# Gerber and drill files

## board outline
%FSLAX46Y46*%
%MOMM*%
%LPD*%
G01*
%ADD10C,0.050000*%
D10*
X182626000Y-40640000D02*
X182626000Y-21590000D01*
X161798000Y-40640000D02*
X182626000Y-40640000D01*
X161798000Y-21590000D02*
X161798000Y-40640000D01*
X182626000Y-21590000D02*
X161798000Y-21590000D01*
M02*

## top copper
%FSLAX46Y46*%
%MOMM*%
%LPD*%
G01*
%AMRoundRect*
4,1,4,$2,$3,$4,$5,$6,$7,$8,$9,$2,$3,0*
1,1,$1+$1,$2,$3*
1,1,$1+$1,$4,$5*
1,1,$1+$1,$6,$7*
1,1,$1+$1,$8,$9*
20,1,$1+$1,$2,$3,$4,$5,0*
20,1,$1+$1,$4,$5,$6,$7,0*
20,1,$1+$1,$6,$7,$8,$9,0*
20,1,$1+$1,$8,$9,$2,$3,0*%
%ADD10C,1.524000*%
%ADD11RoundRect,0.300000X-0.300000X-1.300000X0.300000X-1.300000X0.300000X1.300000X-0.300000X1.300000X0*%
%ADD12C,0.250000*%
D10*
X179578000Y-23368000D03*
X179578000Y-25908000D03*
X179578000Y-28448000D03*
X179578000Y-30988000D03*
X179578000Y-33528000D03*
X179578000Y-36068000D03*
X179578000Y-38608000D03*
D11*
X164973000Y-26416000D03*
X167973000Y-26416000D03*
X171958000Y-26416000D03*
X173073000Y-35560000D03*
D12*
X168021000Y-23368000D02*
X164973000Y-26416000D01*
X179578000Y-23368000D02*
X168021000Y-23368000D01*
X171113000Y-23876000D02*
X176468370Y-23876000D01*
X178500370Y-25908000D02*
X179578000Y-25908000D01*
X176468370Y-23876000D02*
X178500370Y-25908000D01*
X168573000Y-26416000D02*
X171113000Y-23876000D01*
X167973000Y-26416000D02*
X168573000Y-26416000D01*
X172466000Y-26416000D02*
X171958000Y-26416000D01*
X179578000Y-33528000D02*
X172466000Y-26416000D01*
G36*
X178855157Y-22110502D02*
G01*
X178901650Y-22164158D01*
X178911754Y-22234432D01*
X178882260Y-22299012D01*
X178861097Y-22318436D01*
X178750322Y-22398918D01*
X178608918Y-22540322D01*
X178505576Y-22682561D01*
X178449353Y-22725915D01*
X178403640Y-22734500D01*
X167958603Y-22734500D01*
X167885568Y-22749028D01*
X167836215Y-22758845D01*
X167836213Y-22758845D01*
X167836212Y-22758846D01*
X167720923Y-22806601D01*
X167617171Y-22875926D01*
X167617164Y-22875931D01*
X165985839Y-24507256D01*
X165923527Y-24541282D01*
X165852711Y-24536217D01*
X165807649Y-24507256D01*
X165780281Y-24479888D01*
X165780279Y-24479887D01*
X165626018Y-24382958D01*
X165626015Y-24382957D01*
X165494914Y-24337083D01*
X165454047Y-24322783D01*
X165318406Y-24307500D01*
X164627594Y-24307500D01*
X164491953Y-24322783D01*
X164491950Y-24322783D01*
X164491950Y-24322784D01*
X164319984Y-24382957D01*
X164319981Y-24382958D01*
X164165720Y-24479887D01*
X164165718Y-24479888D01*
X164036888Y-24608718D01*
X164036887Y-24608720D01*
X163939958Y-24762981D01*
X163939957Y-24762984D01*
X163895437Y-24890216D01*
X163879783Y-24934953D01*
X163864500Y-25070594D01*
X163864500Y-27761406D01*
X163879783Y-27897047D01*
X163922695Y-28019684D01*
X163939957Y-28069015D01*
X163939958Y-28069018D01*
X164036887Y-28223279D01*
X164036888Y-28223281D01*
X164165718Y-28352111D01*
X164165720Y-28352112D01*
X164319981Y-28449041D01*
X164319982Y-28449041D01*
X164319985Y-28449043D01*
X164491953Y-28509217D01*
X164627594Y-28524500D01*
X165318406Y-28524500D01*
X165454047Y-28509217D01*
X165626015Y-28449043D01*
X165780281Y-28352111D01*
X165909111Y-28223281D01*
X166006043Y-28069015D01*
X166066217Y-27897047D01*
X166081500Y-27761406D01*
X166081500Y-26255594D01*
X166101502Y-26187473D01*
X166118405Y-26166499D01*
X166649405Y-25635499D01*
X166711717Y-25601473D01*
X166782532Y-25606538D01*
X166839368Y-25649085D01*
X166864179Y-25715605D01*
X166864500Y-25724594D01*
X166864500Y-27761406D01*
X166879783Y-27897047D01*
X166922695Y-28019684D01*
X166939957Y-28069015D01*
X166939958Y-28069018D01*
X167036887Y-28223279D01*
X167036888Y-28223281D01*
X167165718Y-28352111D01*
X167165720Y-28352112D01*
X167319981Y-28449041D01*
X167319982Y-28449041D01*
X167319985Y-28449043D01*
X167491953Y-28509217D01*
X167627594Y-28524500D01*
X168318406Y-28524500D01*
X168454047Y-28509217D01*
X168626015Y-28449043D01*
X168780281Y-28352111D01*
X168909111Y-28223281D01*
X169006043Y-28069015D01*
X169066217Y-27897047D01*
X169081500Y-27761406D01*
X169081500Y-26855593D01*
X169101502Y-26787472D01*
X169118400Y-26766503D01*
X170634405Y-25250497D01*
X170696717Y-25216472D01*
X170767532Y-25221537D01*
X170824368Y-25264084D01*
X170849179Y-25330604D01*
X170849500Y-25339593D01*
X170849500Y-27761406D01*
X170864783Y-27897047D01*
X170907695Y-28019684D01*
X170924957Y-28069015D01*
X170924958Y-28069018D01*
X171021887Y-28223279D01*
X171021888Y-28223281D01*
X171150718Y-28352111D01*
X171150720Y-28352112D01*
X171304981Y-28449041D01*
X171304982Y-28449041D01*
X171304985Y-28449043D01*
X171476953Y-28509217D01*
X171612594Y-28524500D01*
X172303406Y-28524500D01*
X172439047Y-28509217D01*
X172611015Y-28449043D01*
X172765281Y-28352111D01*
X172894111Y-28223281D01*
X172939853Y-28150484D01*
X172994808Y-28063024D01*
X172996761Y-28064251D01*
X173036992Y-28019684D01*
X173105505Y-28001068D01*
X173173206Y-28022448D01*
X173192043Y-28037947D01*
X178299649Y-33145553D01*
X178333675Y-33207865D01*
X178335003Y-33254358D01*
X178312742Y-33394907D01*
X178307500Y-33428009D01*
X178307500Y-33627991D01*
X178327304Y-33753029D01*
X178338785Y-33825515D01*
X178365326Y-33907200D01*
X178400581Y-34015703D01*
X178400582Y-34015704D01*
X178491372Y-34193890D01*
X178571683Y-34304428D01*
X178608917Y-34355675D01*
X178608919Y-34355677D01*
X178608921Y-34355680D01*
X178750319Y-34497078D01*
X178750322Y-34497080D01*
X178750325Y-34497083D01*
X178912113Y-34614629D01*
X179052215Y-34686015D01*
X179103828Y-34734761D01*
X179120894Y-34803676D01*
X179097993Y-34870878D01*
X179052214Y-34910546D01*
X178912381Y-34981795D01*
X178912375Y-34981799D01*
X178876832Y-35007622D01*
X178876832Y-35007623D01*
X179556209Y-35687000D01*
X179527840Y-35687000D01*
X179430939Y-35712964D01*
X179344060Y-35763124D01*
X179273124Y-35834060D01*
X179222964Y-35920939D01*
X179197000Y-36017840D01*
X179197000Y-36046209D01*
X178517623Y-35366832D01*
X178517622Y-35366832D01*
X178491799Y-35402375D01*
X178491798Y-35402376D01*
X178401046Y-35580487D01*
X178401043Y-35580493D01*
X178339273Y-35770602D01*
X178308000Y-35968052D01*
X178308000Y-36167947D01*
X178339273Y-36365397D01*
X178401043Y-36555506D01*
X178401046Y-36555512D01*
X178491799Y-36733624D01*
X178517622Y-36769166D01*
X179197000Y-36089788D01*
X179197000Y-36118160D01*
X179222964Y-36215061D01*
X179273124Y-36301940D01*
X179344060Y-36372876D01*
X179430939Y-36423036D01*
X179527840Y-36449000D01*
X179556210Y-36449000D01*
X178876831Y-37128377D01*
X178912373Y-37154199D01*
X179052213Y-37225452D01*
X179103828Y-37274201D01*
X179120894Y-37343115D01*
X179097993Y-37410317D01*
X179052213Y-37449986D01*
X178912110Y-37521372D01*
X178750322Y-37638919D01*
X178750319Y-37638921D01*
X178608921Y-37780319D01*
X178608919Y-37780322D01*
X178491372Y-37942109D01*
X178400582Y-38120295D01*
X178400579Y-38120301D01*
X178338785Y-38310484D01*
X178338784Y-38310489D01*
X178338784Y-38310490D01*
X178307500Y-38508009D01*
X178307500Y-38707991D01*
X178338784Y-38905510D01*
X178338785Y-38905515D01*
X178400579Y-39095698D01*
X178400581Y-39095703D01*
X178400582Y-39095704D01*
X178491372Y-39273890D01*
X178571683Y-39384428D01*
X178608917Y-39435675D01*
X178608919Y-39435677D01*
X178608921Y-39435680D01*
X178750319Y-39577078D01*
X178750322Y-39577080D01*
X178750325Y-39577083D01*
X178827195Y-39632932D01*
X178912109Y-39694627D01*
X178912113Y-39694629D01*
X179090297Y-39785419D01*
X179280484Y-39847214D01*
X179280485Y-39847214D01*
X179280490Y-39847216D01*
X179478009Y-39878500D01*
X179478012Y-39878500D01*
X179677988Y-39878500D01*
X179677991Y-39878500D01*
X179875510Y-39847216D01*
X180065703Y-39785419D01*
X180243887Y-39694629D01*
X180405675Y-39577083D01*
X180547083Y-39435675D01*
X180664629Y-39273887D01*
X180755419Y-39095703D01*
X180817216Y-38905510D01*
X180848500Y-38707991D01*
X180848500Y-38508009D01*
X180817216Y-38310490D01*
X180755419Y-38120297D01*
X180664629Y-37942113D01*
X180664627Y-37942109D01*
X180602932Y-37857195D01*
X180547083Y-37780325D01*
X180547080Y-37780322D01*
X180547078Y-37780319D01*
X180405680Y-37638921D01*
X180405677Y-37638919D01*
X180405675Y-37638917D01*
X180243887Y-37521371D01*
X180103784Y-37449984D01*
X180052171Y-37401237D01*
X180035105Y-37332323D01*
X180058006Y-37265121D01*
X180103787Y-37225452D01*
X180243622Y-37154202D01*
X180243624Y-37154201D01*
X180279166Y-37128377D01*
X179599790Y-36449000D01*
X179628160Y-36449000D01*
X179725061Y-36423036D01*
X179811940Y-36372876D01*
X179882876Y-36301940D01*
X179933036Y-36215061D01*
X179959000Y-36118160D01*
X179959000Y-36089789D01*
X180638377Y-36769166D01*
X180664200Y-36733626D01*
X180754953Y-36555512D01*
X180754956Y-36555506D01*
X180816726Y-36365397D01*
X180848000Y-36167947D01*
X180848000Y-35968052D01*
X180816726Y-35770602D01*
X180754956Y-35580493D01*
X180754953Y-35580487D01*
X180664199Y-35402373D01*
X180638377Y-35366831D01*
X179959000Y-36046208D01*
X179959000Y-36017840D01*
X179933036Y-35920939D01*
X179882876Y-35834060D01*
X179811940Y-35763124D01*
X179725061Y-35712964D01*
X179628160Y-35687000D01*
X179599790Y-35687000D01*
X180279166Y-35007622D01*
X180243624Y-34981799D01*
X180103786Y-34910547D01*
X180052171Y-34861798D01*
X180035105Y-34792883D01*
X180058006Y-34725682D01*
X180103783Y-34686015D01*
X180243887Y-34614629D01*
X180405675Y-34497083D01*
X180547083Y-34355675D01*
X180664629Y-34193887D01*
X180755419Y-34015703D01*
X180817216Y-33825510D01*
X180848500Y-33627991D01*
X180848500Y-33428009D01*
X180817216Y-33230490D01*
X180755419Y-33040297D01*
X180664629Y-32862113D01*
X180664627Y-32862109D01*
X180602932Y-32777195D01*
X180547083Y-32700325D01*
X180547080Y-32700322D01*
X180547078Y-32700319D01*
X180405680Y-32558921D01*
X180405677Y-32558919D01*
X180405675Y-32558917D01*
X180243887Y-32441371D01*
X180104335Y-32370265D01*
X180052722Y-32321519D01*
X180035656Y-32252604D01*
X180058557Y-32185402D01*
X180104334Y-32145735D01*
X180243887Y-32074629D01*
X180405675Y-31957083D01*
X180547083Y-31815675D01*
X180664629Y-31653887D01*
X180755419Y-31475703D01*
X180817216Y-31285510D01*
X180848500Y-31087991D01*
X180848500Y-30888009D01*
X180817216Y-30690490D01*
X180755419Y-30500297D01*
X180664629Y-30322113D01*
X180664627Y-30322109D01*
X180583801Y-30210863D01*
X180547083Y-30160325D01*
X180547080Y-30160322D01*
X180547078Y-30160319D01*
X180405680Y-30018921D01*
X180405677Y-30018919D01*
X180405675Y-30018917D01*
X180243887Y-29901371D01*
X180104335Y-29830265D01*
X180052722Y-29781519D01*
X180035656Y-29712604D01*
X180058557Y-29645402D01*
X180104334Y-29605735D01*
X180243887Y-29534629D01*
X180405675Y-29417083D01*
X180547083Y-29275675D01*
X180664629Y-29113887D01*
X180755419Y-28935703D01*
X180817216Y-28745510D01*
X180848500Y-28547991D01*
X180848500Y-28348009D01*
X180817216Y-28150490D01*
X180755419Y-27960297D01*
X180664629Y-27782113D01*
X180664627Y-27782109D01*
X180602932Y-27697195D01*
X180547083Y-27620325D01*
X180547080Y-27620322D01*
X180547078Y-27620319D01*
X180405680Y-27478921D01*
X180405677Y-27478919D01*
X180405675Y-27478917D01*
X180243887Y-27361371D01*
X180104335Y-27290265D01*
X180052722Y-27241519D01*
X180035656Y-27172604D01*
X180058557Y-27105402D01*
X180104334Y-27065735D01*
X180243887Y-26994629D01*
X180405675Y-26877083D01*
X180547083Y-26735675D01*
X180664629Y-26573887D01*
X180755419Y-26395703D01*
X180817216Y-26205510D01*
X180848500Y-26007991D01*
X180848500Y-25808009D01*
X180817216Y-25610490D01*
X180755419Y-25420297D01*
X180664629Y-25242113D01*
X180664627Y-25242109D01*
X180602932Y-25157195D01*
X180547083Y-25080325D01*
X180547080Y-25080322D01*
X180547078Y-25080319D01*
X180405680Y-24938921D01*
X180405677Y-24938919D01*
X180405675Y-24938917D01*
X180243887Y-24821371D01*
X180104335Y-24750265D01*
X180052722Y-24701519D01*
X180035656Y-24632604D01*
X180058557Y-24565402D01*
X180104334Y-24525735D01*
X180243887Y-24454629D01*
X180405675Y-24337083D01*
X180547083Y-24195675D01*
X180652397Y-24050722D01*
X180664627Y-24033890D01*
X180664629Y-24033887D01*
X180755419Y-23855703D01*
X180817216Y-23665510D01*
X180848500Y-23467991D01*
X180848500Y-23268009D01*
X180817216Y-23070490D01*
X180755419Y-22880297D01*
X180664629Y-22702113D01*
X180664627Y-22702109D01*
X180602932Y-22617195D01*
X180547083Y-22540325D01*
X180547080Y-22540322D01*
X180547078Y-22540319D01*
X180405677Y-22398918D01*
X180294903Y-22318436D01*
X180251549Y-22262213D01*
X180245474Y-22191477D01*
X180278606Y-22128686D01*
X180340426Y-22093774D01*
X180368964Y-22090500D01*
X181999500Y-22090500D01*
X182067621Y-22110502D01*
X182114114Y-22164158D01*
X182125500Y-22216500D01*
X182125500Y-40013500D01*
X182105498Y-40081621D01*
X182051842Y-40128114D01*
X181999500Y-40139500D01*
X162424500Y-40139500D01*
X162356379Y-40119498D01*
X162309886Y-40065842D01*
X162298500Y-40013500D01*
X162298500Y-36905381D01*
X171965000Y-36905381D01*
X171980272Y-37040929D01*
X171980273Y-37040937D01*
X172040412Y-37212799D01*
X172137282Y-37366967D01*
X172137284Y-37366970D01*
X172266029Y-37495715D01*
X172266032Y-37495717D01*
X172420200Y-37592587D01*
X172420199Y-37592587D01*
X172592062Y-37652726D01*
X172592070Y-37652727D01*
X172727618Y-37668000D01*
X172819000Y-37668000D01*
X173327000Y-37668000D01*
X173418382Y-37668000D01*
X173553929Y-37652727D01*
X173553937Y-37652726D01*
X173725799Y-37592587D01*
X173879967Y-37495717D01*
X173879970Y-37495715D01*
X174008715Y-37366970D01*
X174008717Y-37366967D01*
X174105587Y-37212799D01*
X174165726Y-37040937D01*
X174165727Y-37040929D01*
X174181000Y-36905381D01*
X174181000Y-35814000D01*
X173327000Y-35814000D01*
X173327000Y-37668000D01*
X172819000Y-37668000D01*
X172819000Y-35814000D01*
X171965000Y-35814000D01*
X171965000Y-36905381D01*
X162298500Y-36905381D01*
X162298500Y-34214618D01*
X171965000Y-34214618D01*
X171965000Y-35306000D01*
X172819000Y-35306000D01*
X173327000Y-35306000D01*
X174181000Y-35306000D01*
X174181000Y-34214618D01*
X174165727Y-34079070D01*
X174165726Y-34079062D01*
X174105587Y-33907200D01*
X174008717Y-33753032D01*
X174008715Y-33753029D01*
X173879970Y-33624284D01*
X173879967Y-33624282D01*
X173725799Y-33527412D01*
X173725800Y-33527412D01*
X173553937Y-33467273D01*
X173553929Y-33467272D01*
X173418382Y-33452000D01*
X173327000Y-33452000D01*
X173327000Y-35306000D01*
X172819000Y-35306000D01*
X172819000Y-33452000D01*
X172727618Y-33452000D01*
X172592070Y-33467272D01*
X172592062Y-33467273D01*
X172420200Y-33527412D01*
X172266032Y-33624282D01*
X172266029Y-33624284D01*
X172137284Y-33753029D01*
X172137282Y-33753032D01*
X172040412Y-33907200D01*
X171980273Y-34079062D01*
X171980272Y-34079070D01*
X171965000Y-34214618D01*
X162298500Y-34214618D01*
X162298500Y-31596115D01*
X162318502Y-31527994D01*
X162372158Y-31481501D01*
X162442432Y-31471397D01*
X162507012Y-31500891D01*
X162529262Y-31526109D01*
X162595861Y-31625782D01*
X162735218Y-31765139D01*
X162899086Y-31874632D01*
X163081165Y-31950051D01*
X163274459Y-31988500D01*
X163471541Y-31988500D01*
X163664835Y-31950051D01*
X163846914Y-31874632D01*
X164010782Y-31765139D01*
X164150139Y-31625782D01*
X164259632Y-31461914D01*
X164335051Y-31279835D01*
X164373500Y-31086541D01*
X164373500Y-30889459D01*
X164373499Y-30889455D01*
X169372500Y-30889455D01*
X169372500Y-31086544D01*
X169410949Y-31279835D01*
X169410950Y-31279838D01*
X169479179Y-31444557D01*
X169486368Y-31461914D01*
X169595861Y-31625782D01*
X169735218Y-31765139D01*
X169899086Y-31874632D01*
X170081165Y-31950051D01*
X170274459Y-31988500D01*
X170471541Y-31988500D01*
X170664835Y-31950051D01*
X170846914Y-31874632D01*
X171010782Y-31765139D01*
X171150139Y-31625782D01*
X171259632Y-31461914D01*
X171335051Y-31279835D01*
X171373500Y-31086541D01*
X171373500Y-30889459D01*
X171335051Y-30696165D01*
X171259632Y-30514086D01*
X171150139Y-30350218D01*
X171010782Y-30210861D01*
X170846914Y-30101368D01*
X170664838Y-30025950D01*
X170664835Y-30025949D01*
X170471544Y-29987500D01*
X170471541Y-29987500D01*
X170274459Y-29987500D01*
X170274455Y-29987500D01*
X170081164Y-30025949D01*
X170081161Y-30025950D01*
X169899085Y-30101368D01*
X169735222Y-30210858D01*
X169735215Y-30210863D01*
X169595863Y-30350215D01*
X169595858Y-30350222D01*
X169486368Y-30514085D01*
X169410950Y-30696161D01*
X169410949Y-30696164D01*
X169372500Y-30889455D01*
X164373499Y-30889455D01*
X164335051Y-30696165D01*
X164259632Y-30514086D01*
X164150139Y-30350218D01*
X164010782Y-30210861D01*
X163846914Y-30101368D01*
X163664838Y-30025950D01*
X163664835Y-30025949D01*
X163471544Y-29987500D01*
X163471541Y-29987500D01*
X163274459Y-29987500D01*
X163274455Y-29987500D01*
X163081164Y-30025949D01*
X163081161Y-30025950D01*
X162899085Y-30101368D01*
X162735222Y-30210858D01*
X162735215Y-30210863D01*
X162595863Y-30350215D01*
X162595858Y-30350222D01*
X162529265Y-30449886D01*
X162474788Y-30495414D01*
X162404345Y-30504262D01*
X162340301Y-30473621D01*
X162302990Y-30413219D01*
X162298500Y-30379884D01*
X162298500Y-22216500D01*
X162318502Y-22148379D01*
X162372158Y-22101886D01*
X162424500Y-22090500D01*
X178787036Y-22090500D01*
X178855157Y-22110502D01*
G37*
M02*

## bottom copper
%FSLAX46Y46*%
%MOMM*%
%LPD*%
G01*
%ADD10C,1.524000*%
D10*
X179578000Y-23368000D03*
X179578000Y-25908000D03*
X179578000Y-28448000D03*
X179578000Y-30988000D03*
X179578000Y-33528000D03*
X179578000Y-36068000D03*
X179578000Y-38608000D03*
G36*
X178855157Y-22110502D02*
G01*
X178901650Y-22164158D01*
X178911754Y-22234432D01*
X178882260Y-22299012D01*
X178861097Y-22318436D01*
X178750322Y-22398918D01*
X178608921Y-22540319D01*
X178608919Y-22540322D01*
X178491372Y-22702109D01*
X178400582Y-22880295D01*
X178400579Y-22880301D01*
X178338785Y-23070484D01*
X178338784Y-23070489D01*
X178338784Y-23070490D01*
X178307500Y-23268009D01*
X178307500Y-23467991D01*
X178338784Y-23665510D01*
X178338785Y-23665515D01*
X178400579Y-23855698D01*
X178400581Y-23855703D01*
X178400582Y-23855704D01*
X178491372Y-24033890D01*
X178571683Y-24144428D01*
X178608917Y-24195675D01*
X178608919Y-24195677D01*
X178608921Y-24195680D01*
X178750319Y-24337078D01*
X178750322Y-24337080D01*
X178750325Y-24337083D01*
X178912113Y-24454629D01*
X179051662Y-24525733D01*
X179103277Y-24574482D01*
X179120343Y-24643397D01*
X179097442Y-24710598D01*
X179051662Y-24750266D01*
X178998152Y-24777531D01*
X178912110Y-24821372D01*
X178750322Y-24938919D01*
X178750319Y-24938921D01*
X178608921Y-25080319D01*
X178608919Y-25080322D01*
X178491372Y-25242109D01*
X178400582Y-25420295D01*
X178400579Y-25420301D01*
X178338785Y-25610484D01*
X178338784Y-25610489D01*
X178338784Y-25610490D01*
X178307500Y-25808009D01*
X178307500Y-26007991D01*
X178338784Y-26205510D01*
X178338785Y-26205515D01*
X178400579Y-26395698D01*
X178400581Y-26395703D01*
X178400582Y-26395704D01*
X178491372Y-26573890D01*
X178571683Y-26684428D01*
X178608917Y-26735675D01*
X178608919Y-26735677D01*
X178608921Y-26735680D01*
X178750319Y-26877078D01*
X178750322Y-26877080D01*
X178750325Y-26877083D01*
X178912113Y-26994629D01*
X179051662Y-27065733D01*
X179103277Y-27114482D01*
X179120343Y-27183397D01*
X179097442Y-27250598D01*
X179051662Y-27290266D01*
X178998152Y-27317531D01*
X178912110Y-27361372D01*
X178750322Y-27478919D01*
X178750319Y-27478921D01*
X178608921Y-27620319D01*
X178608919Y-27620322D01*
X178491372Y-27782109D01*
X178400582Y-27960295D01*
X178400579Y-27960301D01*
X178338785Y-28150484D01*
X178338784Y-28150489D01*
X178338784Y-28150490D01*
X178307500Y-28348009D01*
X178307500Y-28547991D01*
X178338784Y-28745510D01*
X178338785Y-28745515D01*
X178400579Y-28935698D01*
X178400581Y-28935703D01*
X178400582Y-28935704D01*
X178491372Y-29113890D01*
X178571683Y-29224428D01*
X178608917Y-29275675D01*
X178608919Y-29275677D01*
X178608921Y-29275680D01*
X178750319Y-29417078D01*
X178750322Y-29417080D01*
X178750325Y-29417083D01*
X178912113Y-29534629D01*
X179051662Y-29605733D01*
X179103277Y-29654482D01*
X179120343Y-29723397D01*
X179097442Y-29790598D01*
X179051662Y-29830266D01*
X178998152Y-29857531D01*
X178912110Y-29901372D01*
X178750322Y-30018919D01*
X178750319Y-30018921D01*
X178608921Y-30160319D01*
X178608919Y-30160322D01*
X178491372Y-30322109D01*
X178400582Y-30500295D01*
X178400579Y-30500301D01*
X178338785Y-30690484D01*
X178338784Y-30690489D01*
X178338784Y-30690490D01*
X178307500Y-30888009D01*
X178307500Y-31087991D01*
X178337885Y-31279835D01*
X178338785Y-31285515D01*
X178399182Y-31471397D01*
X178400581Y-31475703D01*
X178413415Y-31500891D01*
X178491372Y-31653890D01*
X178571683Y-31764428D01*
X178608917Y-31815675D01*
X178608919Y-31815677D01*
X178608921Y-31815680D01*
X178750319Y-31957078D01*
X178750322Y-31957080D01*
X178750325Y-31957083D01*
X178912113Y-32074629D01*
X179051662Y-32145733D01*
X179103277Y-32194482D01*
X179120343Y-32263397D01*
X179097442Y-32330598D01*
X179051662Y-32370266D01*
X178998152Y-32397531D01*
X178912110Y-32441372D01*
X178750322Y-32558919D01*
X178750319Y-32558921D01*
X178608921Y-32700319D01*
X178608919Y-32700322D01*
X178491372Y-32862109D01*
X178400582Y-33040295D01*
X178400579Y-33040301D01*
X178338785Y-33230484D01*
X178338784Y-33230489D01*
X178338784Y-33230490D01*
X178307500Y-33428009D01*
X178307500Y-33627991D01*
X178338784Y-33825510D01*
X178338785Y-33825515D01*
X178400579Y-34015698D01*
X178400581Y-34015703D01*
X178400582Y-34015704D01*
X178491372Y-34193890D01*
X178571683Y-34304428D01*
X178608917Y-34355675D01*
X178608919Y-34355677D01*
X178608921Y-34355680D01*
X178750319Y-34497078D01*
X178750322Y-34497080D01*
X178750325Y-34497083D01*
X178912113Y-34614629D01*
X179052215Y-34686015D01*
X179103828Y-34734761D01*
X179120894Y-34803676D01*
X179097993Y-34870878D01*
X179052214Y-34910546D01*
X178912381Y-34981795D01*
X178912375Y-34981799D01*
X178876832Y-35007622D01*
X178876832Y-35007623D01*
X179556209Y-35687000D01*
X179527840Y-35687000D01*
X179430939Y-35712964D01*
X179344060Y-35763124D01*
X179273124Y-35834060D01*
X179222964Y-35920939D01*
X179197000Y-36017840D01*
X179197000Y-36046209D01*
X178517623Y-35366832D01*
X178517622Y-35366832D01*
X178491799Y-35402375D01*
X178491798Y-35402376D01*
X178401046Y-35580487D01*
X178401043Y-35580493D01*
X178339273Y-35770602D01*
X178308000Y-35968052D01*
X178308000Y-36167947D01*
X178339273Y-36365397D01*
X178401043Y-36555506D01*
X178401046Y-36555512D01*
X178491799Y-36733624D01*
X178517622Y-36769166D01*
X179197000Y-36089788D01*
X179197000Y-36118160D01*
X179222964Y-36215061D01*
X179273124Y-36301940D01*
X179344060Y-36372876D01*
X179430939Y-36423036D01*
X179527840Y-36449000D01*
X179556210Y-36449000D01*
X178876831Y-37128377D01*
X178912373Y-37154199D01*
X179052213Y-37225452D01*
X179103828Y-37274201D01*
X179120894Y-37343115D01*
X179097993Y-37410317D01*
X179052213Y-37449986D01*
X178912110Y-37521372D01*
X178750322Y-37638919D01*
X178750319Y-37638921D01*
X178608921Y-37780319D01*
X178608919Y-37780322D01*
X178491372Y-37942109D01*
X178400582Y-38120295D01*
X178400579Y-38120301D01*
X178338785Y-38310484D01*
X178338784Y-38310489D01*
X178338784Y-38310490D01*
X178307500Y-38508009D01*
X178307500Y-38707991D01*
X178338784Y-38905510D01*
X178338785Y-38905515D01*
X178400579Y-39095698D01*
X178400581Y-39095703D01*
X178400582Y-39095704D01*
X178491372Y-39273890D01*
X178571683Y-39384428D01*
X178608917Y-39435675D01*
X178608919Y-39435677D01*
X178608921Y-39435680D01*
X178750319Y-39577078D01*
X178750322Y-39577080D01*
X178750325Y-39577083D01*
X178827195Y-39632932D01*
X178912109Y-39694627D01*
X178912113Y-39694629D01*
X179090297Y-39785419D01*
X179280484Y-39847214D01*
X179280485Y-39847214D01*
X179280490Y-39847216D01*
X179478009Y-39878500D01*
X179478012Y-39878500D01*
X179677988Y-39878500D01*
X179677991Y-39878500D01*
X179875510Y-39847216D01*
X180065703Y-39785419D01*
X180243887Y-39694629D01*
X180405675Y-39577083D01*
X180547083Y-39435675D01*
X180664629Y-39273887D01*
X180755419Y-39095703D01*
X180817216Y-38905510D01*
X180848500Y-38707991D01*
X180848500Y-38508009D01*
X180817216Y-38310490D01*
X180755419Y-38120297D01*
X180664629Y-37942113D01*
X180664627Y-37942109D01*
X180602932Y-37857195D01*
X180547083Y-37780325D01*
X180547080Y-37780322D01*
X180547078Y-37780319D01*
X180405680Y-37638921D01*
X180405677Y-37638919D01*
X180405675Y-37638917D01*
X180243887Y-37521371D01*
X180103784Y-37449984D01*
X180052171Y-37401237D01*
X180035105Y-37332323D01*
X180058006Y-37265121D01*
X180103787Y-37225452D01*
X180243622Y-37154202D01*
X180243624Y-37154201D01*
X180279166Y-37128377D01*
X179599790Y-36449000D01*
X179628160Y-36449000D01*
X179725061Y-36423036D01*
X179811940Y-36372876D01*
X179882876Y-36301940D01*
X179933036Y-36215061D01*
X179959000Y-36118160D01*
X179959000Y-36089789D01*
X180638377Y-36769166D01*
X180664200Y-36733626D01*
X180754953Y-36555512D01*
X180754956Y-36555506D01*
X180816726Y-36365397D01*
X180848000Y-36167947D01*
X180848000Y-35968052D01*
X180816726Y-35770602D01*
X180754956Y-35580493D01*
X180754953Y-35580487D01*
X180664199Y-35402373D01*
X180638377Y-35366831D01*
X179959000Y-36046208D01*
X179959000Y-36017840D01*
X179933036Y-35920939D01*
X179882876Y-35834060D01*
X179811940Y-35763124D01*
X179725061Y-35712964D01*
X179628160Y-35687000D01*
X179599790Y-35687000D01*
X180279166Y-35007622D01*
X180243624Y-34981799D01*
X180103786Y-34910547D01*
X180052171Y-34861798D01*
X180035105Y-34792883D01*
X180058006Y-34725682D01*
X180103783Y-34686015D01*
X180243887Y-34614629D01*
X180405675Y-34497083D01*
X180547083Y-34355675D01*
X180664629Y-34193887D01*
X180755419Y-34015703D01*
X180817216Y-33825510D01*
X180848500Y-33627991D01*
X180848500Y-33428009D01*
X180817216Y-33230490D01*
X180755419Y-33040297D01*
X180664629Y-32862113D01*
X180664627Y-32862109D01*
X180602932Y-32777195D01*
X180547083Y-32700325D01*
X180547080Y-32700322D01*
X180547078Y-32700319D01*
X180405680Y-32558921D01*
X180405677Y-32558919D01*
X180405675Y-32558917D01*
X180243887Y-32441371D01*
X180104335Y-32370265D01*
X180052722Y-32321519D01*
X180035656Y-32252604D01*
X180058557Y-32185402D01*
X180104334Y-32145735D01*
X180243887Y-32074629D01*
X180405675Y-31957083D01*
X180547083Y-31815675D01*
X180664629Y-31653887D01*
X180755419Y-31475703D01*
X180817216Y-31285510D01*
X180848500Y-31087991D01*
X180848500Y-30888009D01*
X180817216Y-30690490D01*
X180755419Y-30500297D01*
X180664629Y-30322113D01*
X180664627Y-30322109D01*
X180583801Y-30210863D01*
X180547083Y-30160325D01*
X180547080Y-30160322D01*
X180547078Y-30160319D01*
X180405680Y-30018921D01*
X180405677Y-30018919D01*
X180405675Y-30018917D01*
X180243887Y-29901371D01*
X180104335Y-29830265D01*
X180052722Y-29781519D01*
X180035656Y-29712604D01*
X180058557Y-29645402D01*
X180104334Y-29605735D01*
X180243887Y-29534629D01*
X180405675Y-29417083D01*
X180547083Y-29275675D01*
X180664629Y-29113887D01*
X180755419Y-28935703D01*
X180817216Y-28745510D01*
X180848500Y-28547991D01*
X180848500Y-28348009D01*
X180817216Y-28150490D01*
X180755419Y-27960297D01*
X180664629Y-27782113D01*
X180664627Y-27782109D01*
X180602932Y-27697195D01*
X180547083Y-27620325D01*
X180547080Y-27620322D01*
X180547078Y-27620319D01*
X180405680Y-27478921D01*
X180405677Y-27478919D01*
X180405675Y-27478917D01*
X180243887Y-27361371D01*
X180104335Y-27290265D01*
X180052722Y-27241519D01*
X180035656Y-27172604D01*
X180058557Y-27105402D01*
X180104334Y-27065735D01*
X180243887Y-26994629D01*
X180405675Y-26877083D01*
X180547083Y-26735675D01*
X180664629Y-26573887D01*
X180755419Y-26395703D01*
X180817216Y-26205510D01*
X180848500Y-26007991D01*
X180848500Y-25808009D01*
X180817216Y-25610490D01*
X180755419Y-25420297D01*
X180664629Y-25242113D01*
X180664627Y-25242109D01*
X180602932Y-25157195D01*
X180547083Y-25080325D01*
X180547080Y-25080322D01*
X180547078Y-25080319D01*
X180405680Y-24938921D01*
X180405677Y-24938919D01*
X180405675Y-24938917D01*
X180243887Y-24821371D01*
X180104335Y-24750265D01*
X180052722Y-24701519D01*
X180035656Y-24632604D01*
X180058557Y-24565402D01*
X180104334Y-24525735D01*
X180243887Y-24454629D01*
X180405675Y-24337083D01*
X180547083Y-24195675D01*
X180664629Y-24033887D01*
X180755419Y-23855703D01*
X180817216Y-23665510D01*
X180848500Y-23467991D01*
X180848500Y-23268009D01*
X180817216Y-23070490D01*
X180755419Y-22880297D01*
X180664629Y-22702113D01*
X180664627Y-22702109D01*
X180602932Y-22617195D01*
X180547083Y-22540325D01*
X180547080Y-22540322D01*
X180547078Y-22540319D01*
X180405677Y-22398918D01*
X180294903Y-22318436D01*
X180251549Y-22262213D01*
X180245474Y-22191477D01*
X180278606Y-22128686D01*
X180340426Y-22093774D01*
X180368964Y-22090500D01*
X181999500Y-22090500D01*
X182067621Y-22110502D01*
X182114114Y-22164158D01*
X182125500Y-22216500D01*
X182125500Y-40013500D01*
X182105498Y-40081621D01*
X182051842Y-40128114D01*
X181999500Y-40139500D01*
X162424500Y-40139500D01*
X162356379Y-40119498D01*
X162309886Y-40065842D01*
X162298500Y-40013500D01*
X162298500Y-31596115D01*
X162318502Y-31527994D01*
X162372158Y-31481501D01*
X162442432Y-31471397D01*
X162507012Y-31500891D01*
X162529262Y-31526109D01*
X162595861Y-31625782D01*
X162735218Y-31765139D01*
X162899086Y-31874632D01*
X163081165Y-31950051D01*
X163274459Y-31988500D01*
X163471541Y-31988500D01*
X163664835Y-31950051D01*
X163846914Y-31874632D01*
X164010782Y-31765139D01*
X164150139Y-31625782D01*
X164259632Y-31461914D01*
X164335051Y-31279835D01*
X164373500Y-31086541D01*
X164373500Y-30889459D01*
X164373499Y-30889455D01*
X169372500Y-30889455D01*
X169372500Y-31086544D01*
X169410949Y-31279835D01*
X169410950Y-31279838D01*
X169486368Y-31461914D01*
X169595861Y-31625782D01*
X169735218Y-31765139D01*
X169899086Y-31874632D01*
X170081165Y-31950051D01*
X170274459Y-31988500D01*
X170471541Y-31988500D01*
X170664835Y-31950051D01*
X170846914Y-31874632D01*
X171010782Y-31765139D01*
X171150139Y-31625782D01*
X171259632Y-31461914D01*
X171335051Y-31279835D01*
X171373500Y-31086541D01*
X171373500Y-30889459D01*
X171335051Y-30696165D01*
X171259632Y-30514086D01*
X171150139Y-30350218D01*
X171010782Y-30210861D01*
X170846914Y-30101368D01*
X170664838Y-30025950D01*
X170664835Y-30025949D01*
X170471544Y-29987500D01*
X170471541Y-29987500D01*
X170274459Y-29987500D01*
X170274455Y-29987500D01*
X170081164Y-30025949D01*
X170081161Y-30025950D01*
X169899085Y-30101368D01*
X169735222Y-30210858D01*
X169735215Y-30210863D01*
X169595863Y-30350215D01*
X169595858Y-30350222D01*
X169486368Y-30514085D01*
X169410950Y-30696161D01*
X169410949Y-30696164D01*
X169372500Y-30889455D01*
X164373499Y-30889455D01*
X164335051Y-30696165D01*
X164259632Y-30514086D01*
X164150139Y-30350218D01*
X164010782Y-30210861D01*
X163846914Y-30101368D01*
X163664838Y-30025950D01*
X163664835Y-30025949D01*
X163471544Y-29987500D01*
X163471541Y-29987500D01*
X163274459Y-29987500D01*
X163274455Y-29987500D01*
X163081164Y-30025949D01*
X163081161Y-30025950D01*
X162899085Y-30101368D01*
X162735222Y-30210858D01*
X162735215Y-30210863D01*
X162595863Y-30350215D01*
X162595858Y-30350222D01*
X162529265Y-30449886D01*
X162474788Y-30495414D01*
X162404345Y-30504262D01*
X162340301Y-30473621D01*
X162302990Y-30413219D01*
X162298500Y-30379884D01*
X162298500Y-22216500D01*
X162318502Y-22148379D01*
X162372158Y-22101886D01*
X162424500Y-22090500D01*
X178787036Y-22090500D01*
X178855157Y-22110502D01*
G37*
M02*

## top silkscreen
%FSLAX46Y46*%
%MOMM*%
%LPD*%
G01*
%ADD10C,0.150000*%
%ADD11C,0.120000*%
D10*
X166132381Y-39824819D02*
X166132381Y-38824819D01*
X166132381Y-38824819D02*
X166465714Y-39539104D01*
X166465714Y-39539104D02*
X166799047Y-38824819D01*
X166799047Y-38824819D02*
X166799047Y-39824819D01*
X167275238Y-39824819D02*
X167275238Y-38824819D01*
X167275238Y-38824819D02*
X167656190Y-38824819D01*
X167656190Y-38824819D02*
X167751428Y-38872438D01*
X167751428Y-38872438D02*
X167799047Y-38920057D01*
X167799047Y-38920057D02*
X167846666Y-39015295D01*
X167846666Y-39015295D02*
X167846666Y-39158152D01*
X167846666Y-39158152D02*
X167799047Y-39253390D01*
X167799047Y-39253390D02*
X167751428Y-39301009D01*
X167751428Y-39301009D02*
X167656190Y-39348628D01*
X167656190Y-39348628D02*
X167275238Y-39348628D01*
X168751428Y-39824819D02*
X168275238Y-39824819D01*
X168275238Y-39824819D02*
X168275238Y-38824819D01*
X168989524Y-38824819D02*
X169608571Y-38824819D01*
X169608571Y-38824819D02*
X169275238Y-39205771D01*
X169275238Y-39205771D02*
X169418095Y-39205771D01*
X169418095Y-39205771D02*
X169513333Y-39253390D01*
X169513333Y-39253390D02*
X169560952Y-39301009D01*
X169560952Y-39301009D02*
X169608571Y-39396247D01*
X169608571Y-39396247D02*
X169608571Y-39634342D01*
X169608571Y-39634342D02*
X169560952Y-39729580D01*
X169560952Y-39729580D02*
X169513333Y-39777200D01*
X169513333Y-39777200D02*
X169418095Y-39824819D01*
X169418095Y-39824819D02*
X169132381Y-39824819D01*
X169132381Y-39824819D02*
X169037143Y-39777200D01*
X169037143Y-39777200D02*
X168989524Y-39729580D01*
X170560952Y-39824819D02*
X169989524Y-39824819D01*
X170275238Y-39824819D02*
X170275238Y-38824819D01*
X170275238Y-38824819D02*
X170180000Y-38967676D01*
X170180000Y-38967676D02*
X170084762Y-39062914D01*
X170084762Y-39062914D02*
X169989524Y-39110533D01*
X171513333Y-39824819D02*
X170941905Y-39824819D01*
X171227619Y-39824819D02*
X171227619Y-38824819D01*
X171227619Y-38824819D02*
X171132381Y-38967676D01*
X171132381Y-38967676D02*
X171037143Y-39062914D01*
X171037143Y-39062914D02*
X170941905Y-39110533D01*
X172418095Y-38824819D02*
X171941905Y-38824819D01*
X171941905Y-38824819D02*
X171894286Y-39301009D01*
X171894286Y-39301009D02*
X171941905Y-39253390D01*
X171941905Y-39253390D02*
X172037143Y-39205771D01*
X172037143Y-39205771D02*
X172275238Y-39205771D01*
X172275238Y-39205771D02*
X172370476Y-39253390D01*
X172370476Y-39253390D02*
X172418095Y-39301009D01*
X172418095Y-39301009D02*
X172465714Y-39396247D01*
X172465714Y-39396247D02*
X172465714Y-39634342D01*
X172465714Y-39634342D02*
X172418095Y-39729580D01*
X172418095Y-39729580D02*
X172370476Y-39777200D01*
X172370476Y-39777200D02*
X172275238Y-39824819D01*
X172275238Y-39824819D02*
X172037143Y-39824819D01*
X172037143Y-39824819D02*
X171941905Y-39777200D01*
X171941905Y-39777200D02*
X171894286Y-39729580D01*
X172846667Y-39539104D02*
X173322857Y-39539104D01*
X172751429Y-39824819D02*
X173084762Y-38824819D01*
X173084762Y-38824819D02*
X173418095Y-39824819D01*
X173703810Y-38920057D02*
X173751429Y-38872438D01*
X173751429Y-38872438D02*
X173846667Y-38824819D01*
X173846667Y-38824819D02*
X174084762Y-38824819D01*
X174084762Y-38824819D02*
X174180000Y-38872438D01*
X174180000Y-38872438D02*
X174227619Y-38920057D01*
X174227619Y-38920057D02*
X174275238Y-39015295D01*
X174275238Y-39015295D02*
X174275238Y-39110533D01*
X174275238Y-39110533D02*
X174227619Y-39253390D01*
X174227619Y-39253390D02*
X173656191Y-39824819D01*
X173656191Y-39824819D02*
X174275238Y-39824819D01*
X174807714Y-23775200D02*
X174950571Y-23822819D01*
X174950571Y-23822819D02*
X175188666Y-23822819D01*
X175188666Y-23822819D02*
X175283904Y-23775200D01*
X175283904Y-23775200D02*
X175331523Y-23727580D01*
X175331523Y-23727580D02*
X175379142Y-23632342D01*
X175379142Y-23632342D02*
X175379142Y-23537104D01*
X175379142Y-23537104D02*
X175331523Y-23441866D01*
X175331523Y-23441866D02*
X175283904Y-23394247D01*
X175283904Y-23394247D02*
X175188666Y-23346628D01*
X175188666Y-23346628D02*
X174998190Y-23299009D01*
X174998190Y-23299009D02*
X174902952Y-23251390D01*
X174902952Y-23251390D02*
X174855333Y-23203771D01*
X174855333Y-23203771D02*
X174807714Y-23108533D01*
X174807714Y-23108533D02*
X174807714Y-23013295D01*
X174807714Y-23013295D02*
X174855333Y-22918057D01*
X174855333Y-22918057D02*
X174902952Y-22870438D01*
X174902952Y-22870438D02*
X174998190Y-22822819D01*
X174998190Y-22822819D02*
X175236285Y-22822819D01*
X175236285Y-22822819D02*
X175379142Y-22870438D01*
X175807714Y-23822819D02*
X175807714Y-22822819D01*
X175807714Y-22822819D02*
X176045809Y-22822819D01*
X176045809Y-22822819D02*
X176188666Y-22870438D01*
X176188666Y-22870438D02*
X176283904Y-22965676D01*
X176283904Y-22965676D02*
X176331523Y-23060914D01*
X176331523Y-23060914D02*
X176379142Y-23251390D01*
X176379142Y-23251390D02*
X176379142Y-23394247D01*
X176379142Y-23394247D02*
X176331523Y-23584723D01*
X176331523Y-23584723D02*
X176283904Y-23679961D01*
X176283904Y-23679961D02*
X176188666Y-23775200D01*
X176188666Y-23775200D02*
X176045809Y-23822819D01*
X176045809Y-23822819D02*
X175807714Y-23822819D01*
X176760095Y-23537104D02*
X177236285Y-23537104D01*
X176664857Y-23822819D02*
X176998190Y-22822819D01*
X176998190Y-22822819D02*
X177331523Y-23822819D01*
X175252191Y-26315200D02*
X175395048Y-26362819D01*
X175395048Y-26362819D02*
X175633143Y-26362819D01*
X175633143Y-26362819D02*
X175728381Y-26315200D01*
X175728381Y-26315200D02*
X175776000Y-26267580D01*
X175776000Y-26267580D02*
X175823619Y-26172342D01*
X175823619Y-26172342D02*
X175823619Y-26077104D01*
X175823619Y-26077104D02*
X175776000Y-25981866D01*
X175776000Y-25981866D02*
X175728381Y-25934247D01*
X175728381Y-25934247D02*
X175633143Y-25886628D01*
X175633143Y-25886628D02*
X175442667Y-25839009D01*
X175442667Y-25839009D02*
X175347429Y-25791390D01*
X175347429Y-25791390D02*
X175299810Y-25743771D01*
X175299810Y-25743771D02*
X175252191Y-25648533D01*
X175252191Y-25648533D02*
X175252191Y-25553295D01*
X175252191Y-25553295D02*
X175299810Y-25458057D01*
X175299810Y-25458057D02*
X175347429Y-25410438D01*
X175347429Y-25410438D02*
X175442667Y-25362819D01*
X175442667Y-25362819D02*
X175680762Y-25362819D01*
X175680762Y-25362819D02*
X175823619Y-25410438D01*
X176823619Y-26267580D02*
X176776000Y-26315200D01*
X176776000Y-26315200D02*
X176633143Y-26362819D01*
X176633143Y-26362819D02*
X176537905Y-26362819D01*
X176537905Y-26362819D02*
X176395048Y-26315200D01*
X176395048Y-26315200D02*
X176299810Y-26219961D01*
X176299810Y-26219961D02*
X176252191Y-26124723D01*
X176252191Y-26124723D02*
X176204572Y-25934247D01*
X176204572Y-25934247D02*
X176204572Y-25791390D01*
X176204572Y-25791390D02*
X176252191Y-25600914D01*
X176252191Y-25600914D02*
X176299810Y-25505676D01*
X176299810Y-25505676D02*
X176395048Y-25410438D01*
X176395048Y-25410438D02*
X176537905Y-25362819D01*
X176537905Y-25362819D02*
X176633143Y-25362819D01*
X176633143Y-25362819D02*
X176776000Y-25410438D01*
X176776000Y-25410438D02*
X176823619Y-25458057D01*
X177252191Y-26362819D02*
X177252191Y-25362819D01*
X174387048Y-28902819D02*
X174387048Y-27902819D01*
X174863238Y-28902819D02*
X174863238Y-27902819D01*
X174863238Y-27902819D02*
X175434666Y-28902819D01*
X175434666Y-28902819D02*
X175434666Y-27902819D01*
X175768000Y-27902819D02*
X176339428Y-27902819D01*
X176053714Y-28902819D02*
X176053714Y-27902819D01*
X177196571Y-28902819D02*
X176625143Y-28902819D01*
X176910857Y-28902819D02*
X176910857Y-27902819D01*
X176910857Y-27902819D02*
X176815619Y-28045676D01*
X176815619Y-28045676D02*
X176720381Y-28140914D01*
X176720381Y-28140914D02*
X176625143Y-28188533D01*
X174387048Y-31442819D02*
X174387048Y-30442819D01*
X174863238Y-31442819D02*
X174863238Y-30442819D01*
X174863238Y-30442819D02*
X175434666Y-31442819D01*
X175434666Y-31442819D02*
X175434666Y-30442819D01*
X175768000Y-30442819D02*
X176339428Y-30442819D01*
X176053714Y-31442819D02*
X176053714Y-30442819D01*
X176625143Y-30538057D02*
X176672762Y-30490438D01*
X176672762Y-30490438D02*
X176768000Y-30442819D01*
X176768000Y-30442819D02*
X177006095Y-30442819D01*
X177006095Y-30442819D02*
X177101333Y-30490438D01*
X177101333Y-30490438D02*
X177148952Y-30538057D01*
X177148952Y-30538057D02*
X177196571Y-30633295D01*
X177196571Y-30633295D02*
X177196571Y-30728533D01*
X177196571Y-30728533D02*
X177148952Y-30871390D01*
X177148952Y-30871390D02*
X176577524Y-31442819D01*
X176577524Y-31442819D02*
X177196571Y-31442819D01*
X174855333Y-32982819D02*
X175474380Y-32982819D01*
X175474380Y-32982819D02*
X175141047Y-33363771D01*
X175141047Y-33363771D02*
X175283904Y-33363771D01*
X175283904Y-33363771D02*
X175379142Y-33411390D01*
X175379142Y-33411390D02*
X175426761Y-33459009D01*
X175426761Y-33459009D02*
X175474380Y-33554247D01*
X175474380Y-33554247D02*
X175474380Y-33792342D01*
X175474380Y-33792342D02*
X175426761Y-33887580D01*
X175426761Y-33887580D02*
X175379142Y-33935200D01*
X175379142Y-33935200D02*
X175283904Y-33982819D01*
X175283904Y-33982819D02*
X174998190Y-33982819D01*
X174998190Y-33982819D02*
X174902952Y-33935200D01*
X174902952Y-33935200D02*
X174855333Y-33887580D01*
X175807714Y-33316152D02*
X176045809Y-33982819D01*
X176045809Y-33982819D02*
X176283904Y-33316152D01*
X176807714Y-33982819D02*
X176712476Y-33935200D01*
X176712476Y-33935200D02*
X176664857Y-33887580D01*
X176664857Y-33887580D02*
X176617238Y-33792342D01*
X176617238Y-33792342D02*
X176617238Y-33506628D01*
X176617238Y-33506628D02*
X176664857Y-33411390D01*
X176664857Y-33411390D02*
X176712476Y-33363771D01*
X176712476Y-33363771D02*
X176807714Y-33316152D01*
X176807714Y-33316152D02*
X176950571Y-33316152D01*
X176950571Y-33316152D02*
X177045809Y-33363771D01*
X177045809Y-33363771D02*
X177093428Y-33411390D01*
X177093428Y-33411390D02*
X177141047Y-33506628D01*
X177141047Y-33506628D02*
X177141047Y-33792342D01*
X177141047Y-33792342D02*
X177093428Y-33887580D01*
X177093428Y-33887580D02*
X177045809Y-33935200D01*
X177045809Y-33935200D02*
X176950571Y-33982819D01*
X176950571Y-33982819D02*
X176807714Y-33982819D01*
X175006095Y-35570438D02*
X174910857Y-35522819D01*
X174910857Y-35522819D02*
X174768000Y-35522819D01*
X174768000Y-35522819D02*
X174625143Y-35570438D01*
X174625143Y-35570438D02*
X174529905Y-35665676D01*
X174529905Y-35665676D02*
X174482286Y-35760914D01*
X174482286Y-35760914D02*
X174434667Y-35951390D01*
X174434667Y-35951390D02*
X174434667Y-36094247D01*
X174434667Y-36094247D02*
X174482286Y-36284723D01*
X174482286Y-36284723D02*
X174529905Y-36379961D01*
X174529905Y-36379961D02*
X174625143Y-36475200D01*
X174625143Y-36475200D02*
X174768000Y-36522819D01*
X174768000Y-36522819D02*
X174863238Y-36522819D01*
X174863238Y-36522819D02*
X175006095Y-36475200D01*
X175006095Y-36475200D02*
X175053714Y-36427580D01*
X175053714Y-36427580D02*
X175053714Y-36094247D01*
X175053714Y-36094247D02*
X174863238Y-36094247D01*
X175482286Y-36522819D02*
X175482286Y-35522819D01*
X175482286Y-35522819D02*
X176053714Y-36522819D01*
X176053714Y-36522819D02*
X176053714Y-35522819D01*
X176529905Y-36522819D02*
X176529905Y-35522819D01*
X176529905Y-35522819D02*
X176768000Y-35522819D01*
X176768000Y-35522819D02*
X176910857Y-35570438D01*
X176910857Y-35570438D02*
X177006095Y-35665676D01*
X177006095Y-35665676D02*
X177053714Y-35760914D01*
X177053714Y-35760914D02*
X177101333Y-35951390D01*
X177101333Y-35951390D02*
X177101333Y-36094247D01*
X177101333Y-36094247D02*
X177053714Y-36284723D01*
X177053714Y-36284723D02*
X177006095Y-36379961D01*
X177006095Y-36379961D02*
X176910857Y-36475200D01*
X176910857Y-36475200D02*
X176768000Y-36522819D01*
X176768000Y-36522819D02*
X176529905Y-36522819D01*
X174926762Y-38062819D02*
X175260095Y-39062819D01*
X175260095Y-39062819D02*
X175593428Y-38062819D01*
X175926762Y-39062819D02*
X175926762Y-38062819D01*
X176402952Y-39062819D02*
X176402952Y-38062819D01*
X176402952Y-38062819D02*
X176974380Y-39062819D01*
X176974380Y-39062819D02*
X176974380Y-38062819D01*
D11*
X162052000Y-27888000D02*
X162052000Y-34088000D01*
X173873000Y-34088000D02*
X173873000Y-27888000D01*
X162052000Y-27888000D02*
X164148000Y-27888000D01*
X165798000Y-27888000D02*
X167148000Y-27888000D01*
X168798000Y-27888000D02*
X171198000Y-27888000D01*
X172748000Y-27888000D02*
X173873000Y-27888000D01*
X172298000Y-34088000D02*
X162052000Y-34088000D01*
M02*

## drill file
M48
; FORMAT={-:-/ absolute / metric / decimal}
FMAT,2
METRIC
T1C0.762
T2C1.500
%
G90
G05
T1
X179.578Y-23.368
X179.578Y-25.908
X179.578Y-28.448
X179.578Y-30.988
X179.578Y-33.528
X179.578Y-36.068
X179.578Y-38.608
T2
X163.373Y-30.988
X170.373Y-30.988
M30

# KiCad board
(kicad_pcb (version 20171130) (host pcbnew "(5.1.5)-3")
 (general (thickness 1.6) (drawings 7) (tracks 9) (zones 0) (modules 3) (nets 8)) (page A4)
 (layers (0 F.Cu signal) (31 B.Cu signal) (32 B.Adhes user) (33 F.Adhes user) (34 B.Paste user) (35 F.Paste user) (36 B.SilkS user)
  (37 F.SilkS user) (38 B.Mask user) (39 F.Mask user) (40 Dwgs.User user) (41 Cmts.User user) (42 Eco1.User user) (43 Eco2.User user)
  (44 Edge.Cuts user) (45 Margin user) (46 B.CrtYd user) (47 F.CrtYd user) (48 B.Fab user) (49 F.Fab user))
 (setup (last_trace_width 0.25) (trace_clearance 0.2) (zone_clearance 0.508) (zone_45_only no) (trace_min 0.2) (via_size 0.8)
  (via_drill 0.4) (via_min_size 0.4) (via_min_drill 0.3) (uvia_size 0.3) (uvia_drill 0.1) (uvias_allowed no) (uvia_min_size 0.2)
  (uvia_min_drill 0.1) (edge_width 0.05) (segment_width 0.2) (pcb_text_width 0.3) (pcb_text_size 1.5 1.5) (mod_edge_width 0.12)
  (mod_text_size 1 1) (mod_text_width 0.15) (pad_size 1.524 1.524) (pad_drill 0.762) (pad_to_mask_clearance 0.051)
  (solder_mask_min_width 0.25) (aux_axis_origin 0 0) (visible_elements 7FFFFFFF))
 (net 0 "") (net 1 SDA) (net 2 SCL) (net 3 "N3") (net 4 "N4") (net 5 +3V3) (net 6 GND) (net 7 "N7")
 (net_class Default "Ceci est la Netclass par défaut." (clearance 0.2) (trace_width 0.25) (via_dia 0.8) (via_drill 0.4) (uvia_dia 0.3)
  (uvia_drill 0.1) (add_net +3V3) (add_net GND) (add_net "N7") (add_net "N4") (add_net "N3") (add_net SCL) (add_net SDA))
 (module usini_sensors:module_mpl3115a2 (layer F.Cu) (at 182.118 28.448 180)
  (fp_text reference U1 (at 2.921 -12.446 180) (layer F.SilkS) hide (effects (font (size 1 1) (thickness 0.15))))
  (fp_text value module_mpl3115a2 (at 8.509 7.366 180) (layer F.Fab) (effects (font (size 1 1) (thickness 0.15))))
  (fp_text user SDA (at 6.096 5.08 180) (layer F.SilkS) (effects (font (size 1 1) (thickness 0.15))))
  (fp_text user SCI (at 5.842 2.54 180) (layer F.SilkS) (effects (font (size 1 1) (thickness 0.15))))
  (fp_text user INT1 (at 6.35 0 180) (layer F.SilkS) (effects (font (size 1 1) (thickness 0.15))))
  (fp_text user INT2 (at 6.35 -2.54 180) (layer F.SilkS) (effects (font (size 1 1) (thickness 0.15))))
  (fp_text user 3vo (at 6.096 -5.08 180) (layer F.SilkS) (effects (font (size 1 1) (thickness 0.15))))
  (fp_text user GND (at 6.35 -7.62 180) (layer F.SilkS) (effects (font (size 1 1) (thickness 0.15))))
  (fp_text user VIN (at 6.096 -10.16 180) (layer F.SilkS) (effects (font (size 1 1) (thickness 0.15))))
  (pad 7 thru_hole circle (at 2.54 5.08 180) (size 1.524 1.524) (drill 0.762) (layers *.Cu *.Mask) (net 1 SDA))
  (pad 6 thru_hole circle (at 2.54 2.54 180) (size 1.524 1.524) (drill 0.762) (layers *.Cu *.Mask) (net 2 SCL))
  (pad 5 thru_hole circle (at 2.54 0 180) (size 1.524 1.524) (drill 0.762) (layers *.Cu *.Mask) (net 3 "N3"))
  (pad 4 thru_hole circle (at 2.54 -2.54 180) (size 1.524 1.524) (drill 0.762) (layers *.Cu *.Mask) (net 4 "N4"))
  (pad 3 thru_hole circle (at 2.54 -5.08 180) (size 1.524 1.524) (drill 0.762) (layers *.Cu *.Mask) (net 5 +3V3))
  (pad 2 thru_hole circle (at 2.54 -7.62 180) (size 1.524 1.524) (drill 0.762) (layers *.Cu *.Mask) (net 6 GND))
  (pad 1 thru_hole circle (at 2.54 -10.16 180) (size 1.524 1.524) (drill 0.762) (layers *.Cu *.Mask) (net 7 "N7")))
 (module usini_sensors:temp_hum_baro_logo (layer B.Cu) (at 174.498 24.384 180)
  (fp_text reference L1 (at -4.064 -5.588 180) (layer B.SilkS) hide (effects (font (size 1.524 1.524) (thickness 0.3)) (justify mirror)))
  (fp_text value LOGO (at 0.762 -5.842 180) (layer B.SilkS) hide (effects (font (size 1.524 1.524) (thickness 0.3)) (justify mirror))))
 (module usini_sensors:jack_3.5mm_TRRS (layer F.Cu) (at 168.148 30.988)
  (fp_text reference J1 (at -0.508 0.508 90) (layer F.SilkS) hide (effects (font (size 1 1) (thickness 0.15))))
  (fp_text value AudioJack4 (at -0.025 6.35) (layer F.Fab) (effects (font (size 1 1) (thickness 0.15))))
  (fp_line (start -6.096 -3.1) (end -6.096 3.1) (layer F.SilkS) (width 0.12))
  (fp_line (start 5.725 3.1) (end 5.725 -3.1) (layer F.SilkS) (width 0.12))
  (fp_line (start -6.096 -3.1) (end -4 -3.1) (layer F.SilkS) (width 0.12))
  (fp_line (start -2.35 -3.1) (end -1 -3.1) (layer F.SilkS) (width 0.12))
  (fp_line (start 0.65 -3.1) (end 3.05 -3.1) (layer F.SilkS) (width 0.12))
  (fp_line (start 4.6 -3.1) (end 5.725 -3.1) (layer F.SilkS) (width 0.12))
  (fp_line (start 4.15 3.1) (end -6.096 3.1) (layer F.SilkS) (width 0.12))
  (pad "" np_thru_hole circle (at 2.225 0) (size 1.5 1.5) (drill 1.5) (layers *.Cu *.Mask))
  (pad "" np_thru_hole circle (at -4.775 0) (size 1.5 1.5) (drill 1.5) (layers *.Cu *.Mask))
  (pad R2 smd roundrect (at -3.175 -4.572) (size 1.2 3.2) (layers F.Cu F.Paste F.Mask) (roundrect_rratio 0.25) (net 1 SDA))
  (pad R1 smd roundrect (at -0.175 -4.572) (size 1.2 3.2) (layers F.Cu F.Paste F.Mask) (roundrect_rratio 0.25) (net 2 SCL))
  (pad T smd roundrect (at 3.81 -4.572) (size 1.2 3.2) (layers F.Cu F.Paste F.Mask) (roundrect_rratio 0.25) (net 5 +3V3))
  (pad S smd roundrect (at 4.925 4.572) (size 1.2 3.2) (layers F.Cu F.Paste F.Mask) (roundrect_rratio 0.25) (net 6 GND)))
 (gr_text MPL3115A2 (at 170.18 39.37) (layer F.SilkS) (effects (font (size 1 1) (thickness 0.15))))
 (gr_line (start 182.626 40.64) (end 182.626 21.59) (layer Edge.Cuts) (width 0.05))
 (gr_line (start 161.798 40.64) (end 182.626 40.64) (layer Edge.Cuts) (width 0.05))
 (gr_line (start 161.798 21.59) (end 161.798 40.64) (layer Edge.Cuts) (width 0.05))
 (gr_line (start 182.626 21.59) (end 161.798 21.59) (layer Edge.Cuts) (width 0.05))
 (segment (start 168.021 23.368) (end 164.973 26.416) (width 0.25) (layer F.Cu) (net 1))
 (segment (start 179.578 23.368) (end 168.021 23.368) (width 0.25) (layer F.Cu) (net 1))
 (segment (start 171.113 23.876) (end 176.46837 23.876) (width 0.25) (layer F.Cu) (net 2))
 (segment (start 178.50037 25.908) (end 179.578 25.908) (width 0.25) (layer F.Cu) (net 2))
 (segment (start 176.46837 23.876) (end 178.50037 25.908) (width 0.25) (layer F.Cu) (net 2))
 (segment (start 168.573 26.416) (end 171.113 23.876) (width 0.25) (layer F.Cu) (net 2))
 (segment (start 167.973 26.416) (end 168.573 26.416) (width 0.25) (layer F.Cu) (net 2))
 (segment (start 172.466 26.416) (end 171.958 26.416) (width 0.25) (layer F.Cu) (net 5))
 (segment (start 179.578 33.528) (end 172.466 26.416) (width 0.25) (layer F.Cu) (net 5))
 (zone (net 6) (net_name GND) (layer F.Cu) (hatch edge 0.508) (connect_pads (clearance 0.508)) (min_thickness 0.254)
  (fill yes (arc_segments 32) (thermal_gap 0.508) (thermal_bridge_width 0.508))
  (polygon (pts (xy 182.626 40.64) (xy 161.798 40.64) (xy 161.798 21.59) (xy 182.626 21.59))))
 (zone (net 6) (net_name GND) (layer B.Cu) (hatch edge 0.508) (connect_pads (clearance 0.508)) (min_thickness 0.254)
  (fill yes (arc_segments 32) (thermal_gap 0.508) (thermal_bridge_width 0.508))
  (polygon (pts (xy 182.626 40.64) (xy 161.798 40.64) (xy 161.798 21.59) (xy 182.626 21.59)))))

